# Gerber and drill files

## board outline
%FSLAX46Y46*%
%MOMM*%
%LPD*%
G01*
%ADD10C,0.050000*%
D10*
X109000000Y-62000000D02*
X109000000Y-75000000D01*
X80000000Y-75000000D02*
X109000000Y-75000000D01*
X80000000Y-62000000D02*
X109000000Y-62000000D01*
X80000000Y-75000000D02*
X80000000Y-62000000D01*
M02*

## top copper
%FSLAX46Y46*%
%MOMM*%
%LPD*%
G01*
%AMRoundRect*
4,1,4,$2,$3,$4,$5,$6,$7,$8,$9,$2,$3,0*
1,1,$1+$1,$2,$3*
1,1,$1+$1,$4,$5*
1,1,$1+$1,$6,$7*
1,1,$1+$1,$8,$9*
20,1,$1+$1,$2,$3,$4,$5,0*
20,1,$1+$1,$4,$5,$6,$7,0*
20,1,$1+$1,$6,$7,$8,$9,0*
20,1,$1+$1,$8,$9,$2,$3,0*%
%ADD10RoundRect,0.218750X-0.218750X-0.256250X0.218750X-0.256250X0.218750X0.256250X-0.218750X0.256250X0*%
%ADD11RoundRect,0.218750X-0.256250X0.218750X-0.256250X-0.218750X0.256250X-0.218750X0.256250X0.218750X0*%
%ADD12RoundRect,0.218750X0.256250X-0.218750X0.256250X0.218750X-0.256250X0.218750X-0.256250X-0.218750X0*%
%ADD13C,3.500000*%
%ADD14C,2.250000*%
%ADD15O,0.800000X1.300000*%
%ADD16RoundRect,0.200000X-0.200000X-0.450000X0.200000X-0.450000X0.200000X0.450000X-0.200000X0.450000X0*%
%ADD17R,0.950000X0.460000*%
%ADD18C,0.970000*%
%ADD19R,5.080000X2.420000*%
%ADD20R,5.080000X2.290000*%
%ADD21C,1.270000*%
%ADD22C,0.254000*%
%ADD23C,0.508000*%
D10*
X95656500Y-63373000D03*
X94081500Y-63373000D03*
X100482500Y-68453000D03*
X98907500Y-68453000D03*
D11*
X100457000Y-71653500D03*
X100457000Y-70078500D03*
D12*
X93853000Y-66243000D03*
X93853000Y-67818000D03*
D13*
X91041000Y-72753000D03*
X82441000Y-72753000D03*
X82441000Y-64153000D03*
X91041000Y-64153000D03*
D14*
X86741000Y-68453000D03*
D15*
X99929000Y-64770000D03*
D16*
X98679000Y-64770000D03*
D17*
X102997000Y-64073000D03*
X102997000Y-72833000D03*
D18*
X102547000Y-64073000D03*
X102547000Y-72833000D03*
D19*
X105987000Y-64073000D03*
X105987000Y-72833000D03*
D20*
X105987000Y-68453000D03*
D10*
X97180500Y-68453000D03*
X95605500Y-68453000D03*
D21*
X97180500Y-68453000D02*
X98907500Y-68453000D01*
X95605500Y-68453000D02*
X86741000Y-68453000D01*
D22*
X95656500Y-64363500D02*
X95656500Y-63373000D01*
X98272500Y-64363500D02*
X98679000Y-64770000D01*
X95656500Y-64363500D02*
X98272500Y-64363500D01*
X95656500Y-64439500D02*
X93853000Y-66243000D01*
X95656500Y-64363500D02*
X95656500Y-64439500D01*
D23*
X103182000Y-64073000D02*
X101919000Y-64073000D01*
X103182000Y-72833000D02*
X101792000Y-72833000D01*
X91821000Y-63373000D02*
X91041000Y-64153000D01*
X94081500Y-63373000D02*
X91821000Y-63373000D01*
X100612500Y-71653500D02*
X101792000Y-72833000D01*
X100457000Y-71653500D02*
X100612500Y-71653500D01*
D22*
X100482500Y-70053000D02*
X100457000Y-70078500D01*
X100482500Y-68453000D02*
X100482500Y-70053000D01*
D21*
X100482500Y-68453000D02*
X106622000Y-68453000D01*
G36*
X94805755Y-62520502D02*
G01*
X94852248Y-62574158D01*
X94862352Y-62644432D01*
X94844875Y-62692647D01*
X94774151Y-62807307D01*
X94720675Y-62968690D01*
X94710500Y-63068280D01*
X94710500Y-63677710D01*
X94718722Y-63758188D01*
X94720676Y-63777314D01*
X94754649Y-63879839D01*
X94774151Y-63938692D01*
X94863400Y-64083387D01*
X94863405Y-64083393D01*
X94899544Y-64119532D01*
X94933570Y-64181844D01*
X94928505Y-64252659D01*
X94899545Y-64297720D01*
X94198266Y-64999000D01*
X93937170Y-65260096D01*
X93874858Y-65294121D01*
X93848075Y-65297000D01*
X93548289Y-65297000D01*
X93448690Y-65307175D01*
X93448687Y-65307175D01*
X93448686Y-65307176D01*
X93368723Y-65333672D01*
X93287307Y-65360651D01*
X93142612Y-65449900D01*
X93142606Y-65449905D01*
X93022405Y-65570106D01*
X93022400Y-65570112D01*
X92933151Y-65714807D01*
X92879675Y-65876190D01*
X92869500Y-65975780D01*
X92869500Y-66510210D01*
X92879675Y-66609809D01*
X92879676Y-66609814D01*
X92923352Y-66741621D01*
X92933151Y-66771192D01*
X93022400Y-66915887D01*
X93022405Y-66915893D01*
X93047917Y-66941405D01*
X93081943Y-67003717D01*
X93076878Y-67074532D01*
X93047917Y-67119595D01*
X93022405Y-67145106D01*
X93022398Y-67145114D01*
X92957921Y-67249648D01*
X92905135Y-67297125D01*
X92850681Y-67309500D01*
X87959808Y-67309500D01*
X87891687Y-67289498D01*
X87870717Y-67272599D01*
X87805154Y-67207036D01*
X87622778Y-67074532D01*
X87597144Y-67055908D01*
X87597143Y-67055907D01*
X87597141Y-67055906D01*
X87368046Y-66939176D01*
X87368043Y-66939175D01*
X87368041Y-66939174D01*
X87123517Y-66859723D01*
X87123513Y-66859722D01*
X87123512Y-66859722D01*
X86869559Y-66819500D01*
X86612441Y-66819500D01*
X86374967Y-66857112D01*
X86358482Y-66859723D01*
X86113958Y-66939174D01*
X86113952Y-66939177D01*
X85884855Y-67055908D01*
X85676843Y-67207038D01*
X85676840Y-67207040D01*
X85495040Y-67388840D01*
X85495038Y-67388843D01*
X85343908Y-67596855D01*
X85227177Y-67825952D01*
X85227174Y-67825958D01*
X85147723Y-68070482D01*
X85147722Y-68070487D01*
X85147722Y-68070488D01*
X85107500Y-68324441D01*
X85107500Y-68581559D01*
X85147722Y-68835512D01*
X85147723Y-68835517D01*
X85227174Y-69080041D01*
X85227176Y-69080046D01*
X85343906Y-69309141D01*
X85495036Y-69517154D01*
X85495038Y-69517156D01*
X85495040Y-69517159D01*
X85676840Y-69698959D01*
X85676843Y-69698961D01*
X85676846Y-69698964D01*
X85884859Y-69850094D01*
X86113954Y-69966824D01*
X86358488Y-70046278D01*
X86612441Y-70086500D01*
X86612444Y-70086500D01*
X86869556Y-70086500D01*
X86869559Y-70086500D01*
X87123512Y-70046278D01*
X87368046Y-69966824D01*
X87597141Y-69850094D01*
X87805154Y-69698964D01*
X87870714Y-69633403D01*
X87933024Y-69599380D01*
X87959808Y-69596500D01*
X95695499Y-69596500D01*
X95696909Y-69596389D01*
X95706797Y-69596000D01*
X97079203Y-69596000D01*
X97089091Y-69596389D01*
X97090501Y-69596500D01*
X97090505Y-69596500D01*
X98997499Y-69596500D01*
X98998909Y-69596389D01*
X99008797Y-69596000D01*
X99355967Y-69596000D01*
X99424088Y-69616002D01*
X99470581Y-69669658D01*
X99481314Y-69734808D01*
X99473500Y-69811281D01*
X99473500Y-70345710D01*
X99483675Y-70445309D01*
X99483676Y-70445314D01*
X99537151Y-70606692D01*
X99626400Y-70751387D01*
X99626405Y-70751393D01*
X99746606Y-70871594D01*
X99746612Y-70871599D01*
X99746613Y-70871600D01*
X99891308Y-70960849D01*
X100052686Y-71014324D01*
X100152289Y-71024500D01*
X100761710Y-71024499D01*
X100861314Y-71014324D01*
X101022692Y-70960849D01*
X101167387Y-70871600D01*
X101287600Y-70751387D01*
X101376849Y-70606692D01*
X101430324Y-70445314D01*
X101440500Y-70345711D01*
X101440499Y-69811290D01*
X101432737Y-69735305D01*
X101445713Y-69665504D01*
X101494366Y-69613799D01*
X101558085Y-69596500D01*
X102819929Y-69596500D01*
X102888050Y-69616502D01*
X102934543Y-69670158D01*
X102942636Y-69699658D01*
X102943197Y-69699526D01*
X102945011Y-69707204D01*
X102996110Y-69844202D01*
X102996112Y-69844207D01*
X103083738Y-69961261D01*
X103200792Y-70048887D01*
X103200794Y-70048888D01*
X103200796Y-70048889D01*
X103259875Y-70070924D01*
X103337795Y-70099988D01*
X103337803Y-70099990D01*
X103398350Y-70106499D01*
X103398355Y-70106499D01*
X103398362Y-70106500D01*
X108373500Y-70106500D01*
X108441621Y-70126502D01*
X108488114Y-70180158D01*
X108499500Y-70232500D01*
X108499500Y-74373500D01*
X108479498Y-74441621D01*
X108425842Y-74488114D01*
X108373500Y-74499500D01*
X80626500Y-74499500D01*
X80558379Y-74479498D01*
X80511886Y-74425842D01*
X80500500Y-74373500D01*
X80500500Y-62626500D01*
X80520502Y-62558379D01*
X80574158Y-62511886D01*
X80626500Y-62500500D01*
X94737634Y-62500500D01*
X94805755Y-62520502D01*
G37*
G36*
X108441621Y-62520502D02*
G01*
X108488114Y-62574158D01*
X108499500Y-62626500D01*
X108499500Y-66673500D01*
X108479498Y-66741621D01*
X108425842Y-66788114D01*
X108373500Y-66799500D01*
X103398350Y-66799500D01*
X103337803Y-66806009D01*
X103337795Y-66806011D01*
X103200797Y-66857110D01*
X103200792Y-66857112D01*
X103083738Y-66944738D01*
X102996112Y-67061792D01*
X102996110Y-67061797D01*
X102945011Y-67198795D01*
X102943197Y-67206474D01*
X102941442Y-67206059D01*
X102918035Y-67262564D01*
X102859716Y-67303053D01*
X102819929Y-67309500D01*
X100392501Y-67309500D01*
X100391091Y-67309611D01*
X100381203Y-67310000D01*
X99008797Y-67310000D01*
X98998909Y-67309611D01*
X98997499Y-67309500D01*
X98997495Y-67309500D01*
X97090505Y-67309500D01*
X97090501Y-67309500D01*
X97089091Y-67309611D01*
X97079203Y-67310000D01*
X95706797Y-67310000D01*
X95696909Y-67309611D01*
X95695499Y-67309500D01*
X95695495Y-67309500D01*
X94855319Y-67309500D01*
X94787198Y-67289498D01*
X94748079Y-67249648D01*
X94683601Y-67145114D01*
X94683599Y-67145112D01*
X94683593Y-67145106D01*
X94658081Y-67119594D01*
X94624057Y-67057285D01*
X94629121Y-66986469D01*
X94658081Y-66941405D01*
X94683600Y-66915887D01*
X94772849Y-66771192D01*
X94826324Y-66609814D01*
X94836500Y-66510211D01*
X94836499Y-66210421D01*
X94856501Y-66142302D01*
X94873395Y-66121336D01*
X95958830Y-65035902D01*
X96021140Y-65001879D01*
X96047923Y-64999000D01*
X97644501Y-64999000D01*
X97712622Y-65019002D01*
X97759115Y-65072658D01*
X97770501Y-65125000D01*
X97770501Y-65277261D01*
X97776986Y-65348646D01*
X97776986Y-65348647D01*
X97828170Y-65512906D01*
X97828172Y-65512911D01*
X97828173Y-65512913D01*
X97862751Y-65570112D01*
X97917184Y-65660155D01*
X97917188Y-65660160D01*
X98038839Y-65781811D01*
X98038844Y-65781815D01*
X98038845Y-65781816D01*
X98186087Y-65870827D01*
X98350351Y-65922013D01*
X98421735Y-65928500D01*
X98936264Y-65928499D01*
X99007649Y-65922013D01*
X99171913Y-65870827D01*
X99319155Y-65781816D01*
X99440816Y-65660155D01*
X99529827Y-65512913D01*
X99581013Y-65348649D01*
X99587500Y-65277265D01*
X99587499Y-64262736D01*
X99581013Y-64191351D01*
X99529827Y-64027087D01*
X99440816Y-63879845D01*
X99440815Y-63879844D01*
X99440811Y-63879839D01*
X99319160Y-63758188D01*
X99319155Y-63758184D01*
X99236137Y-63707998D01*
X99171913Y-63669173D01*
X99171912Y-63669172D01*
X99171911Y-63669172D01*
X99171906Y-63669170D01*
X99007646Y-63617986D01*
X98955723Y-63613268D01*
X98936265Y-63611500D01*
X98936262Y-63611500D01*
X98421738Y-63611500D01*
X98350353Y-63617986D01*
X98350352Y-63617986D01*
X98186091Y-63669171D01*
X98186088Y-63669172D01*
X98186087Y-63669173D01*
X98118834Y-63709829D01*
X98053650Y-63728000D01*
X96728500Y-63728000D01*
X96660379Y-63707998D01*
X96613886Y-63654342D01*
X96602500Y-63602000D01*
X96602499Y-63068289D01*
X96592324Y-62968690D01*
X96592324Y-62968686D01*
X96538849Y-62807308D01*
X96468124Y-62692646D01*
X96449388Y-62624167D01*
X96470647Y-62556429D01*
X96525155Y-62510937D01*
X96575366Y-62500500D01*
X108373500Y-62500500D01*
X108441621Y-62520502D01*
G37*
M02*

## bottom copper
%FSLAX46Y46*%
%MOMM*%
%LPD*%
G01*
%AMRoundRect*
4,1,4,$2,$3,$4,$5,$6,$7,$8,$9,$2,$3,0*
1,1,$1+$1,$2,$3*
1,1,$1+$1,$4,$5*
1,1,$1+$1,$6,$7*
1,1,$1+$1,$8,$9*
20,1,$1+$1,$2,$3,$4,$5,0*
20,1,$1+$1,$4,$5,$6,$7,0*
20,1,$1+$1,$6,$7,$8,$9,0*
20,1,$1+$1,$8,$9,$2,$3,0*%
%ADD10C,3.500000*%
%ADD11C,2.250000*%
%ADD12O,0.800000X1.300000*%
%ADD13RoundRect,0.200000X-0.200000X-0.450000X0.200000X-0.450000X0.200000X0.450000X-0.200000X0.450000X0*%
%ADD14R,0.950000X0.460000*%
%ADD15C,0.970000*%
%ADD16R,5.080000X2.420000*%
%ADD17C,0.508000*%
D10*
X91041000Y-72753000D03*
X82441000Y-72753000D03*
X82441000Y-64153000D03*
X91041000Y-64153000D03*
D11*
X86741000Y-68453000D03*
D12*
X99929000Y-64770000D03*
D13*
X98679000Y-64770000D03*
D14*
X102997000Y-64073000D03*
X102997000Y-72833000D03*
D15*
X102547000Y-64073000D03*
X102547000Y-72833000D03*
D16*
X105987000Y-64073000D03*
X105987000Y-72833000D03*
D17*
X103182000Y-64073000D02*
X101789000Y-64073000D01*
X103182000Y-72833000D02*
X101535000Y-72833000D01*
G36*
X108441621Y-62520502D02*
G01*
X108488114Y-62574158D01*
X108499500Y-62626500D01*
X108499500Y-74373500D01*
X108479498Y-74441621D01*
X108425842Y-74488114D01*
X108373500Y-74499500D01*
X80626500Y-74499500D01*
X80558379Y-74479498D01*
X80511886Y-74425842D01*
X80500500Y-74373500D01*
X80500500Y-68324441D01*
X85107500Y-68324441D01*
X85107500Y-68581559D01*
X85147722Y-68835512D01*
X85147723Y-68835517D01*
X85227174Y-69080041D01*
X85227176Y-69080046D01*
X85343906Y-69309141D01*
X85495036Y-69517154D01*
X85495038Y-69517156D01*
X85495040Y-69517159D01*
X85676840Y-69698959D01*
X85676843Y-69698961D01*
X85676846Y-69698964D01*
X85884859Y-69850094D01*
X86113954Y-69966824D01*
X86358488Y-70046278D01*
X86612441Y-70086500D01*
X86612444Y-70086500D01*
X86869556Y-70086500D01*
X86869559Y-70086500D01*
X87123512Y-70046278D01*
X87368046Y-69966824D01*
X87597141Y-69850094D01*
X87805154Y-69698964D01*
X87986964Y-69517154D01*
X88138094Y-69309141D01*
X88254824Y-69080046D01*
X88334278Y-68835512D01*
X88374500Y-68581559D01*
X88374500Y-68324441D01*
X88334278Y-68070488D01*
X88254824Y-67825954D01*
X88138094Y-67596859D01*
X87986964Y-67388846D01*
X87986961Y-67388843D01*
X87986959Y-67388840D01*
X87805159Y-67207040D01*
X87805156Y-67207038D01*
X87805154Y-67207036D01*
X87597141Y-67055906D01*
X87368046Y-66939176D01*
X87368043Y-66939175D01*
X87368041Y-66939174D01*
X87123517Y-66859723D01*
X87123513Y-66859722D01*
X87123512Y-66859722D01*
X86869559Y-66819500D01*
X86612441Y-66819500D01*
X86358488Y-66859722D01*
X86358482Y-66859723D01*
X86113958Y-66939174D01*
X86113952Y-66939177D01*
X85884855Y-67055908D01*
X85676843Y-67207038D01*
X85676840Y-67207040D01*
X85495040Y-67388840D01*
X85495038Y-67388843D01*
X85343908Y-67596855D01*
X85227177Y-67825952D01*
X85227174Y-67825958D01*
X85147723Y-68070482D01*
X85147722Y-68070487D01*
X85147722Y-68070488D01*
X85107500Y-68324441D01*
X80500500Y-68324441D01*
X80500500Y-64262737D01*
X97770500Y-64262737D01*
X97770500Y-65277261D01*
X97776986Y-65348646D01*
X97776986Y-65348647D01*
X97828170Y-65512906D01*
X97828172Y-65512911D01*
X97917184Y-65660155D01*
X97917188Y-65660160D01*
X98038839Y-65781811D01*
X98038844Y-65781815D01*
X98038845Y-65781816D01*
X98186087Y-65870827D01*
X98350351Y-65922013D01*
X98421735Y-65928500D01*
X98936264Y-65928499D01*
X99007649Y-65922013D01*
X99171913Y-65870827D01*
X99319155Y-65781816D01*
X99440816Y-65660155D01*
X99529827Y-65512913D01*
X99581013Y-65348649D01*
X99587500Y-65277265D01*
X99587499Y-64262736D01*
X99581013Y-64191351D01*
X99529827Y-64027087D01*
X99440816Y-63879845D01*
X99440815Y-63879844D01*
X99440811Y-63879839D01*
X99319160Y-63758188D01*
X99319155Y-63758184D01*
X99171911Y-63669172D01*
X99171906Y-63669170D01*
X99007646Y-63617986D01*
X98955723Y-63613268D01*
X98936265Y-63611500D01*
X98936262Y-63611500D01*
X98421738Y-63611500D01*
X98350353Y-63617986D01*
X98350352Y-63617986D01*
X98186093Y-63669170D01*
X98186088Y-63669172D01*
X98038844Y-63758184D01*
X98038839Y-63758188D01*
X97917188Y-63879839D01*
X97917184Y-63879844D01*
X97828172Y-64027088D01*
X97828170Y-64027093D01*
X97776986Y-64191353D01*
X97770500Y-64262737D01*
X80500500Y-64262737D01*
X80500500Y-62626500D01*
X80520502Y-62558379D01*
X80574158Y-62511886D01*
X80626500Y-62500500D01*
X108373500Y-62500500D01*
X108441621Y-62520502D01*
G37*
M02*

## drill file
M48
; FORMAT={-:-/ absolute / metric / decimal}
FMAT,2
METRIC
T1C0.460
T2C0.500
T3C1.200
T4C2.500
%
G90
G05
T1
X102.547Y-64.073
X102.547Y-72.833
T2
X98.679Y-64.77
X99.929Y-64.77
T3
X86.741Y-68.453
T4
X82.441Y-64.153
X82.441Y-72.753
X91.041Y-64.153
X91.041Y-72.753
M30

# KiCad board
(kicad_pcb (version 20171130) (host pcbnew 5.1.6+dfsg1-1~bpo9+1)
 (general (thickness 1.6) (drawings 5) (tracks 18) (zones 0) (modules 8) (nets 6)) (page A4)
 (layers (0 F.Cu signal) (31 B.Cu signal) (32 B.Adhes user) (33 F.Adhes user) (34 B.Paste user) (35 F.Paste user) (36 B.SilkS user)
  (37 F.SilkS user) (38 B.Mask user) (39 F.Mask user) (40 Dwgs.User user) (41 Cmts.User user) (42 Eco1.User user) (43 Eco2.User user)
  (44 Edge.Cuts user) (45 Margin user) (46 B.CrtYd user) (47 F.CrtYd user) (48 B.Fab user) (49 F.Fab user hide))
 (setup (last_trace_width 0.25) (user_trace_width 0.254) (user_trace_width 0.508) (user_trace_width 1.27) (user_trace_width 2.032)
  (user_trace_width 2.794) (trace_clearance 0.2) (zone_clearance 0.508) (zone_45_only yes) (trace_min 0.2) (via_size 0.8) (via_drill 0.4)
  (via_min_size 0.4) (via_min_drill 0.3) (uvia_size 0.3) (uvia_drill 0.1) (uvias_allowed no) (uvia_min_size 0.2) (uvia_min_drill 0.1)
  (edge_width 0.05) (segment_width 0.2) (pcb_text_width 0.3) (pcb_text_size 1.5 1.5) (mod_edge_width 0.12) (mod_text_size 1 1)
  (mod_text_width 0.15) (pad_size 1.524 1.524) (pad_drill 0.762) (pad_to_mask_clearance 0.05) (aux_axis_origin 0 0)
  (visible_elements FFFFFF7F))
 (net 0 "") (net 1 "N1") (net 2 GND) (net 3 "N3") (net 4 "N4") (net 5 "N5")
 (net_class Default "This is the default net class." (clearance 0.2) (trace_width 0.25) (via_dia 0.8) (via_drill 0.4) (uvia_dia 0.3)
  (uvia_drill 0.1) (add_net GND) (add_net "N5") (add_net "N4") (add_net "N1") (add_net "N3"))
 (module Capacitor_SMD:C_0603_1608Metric (layer F.Cu) (at 94.869 63.373)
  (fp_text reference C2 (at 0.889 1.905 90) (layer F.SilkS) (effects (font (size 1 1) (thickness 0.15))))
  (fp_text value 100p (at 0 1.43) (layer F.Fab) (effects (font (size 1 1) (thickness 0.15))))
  (pad 2 smd roundrect (at 0.7875 0) (size 0.875 0.95) (layers F.Cu F.Paste F.Mask) (roundrect_rratio 0.25) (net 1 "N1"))
  (pad 1 smd roundrect (at -0.7875 0) (size 0.875 0.95) (layers F.Cu F.Paste F.Mask) (roundrect_rratio 0.25) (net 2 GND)))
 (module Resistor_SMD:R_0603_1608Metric (layer F.Cu) (at 99.695 68.453)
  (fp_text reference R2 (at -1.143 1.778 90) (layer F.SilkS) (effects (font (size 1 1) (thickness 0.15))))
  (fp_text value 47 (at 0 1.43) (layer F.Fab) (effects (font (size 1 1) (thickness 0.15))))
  (pad 2 smd roundrect (at 0.7875 0) (size 0.875 0.95) (layers F.Cu F.Paste F.Mask) (roundrect_rratio 0.25) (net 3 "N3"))
  (pad 1 smd roundrect (at -0.7875 0) (size 0.875 0.95) (layers F.Cu F.Paste F.Mask) (roundrect_rratio 0.25) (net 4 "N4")))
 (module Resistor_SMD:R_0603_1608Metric (layer F.Cu) (at 100.457 70.866 270)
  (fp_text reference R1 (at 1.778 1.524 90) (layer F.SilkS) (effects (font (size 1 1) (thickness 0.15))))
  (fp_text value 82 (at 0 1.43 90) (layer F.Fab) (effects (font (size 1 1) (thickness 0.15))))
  (pad 2 smd roundrect (at 0.7875 0 270) (size 0.875 0.95) (layers F.Cu F.Paste F.Mask) (roundrect_rratio 0.25) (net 2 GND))
  (pad 1 smd roundrect (at -0.7875 0 270) (size 0.875 0.95) (layers F.Cu F.Paste F.Mask) (roundrect_rratio 0.25) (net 3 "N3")))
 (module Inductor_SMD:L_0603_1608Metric (layer F.Cu) (at 93.853 67.0305 90)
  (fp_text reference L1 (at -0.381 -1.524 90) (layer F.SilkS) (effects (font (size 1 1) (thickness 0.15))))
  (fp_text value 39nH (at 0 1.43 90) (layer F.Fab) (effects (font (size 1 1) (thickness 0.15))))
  (pad 2 smd roundrect (at 0.7875 0 90) (size 0.875 0.95) (layers F.Cu F.Paste F.Mask) (roundrect_rratio 0.25) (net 1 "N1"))
  (pad 1 smd roundrect (at -0.7875 0 90) (size 0.875 0.95) (layers F.Cu F.Paste F.Mask) (roundrect_rratio 0.25) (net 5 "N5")))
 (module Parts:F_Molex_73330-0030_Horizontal (layer F.Cu) (at 86.741 68.453 90)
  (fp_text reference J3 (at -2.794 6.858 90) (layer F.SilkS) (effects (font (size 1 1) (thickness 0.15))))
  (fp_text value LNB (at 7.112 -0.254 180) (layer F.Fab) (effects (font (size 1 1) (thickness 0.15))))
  (pad 2 thru_hole circle (at -4.3 4.3 90) (size 3.5 3.5) (drill 2.5) (layers *.Cu *.Mask) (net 2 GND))
  (pad 2 thru_hole circle (at -4.3 -4.3 90) (size 3.5 3.5) (drill 2.5) (layers *.Cu *.Mask) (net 2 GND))
  (pad 2 thru_hole circle (at 4.3 -4.3 90) (size 3.5 3.5) (drill 2.5) (layers *.Cu *.Mask) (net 2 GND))
  (pad 2 thru_hole circle (at 4.3 4.3 180) (size 3.5 3.5) (drill 2.5) (layers *.Cu *.Mask) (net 2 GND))
  (pad 1 thru_hole circle (at 0 0 90) (size 2.25 2.25) (drill 1.2) (layers *.Cu *.Mask) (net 5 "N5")))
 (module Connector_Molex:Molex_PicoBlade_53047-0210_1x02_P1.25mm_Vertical (layer F.Cu) (at 98.679 64.77)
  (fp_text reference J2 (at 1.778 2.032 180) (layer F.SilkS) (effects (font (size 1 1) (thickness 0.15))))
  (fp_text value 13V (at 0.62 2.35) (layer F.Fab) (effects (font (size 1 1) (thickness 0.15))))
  (pad 2 thru_hole oval (at 1.25 0) (size 0.8 1.3) (drill 0.5) (layers *.Cu *.Mask) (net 2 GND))
  (pad 1 thru_hole roundrect (at 0 0) (size 0.8 1.3) (drill 0.5) (layers *.Cu *.Mask) (roundrect_rratio 0.25) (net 1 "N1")))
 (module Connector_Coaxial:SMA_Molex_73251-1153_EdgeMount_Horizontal (layer F.Cu) (at 104.267 68.453 180)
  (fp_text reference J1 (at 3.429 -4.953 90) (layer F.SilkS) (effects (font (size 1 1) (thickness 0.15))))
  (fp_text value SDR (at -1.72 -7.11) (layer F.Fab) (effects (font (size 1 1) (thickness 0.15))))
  (pad 2 smd rect (at 1.27 4.38 180) (size 0.95 0.46) (layers B.Cu) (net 2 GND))
  (pad 2 smd rect (at 1.27 -4.38 180) (size 0.95 0.46) (layers B.Cu) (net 2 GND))
  (pad 2 smd rect (at 1.27 4.38 180) (size 0.95 0.46) (layers F.Cu) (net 2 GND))
  (pad 2 smd rect (at 1.27 -4.38 180) (size 0.95 0.46) (layers F.Cu) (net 2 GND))
  (pad 2 thru_hole circle (at 1.72 4.38 180) (size 0.97 0.97) (drill 0.46) (layers *.Cu) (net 2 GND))
  (pad 2 thru_hole circle (at 1.72 -4.38 180) (size 0.97 0.97) (drill 0.46) (layers *.Cu) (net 2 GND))
  (pad 2 smd rect (at -1.72 4.38 180) (size 5.08 2.42) (layers B.Cu B.Paste B.Mask) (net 2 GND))
  (pad 2 smd rect (at -1.72 -4.38 180) (size 5.08 2.42) (layers B.Cu B.Paste B.Mask) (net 2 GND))
  (pad 2 smd rect (at -1.72 4.38 180) (size 5.08 2.42) (layers F.Cu F.Paste F.Mask) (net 2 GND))
  (pad 2 smd rect (at -1.72 -4.38 180) (size 5.08 2.42) (layers F.Cu F.Paste F.Mask) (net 2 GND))
  (pad 1 smd rect (at -1.72 0 180) (size 5.08 2.29) (layers F.Cu F.Paste F.Mask) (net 3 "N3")))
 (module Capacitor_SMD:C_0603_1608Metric (layer F.Cu) (at 96.393 68.453)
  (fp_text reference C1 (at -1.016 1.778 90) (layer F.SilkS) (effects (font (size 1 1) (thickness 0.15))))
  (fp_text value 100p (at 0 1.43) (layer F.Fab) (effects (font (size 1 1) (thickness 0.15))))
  (pad 2 smd roundrect (at 0.7875 0) (size 0.875 0.95) (layers F.Cu F.Paste F.Mask) (roundrect_rratio 0.25) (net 4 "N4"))
  (pad 1 smd roundrect (at -0.7875 0) (size 0.875 0.95) (layers F.Cu F.Paste F.Mask) (roundrect_rratio 0.25) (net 5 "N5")))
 (gr_line (start 109 62) (end 109 75) (layer Edge.Cuts) (width 0.05))
 (gr_line (start 80 75) (end 109 75) (layer Edge.Cuts) (width 0.05))
 (gr_line (start 80 62) (end 109 62) (layer Edge.Cuts) (width 0.05))
 (gr_line (start 80 75) (end 80 62) (layer Edge.Cuts) (width 0.05))
 (segment (start 97.1805 68.453) (end 98.9075 68.453) (width 1.27) (layer F.Cu) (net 4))
 (segment (start 95.6055 68.453) (end 86.741 68.453) (width 1.27) (layer F.Cu) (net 5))
 (segment (start 95.6565 64.3635) (end 95.6565 63.373) (width 0.254) (layer F.Cu) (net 1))
 (segment (start 98.2725 64.3635) (end 98.679 64.77) (width 0.254) (layer F.Cu) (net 1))
 (segment (start 95.6565 64.3635) (end 98.2725 64.3635) (width 0.254) (layer F.Cu) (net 1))
 (segment (start 95.6565 64.4395) (end 93.853 66.243) (width 0.254) (layer F.Cu) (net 1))
 (segment (start 95.6565 64.3635) (end 95.6565 64.4395) (width 0.254) (layer F.Cu) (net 1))
 (segment (start 103.182 64.073) (end 101.919 64.073) (width 0.508) (layer F.Cu) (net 2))
 (segment (start 103.182 64.073) (end 101.789 64.073) (width 0.508) (layer B.Cu) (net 2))
 (segment (start 103.182 72.833) (end 101.535 72.833) (width 0.508) (layer B.Cu) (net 2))
 (segment (start 103.182 72.833) (end 101.792 72.833) (width 0.508) (layer F.Cu) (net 2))
 (segment (start 91.821 63.373) (end 91.041 64.153) (width 0.508) (layer F.Cu) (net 2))
 (segment (start 94.0815 63.373) (end 91.821 63.373) (width 0.508) (layer F.Cu) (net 2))
 (segment (start 100.6125 71.6535) (end 101.792 72.833) (width 0.508) (layer F.Cu) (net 2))
 (segment (start 100.457 71.6535) (end 100.6125 71.6535) (width 0.508) (layer F.Cu) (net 2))
 (segment (start 100.4825 70.053) (end 100.457 70.0785) (width 0.254) (layer F.Cu) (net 3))
 (segment (start 100.4825 68.453) (end 100.4825 70.053) (width 0.254) (layer F.Cu) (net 3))
 (segment (start 100.4825 68.453) (end 106.622 68.453) (width 1.27) (layer F.Cu) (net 3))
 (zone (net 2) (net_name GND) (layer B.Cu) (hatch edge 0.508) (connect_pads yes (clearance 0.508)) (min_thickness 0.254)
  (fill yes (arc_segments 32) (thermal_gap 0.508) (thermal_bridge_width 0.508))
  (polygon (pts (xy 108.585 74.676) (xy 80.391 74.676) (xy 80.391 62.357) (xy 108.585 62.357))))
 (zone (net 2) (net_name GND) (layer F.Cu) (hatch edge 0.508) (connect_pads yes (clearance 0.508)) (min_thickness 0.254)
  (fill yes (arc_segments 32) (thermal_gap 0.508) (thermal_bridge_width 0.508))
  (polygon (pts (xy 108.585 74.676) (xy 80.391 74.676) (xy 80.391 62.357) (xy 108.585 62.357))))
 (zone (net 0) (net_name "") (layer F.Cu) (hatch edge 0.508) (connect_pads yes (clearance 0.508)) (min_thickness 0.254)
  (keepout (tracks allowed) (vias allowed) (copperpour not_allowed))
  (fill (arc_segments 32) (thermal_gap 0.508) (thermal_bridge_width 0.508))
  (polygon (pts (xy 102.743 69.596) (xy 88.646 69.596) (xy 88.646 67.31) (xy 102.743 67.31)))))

